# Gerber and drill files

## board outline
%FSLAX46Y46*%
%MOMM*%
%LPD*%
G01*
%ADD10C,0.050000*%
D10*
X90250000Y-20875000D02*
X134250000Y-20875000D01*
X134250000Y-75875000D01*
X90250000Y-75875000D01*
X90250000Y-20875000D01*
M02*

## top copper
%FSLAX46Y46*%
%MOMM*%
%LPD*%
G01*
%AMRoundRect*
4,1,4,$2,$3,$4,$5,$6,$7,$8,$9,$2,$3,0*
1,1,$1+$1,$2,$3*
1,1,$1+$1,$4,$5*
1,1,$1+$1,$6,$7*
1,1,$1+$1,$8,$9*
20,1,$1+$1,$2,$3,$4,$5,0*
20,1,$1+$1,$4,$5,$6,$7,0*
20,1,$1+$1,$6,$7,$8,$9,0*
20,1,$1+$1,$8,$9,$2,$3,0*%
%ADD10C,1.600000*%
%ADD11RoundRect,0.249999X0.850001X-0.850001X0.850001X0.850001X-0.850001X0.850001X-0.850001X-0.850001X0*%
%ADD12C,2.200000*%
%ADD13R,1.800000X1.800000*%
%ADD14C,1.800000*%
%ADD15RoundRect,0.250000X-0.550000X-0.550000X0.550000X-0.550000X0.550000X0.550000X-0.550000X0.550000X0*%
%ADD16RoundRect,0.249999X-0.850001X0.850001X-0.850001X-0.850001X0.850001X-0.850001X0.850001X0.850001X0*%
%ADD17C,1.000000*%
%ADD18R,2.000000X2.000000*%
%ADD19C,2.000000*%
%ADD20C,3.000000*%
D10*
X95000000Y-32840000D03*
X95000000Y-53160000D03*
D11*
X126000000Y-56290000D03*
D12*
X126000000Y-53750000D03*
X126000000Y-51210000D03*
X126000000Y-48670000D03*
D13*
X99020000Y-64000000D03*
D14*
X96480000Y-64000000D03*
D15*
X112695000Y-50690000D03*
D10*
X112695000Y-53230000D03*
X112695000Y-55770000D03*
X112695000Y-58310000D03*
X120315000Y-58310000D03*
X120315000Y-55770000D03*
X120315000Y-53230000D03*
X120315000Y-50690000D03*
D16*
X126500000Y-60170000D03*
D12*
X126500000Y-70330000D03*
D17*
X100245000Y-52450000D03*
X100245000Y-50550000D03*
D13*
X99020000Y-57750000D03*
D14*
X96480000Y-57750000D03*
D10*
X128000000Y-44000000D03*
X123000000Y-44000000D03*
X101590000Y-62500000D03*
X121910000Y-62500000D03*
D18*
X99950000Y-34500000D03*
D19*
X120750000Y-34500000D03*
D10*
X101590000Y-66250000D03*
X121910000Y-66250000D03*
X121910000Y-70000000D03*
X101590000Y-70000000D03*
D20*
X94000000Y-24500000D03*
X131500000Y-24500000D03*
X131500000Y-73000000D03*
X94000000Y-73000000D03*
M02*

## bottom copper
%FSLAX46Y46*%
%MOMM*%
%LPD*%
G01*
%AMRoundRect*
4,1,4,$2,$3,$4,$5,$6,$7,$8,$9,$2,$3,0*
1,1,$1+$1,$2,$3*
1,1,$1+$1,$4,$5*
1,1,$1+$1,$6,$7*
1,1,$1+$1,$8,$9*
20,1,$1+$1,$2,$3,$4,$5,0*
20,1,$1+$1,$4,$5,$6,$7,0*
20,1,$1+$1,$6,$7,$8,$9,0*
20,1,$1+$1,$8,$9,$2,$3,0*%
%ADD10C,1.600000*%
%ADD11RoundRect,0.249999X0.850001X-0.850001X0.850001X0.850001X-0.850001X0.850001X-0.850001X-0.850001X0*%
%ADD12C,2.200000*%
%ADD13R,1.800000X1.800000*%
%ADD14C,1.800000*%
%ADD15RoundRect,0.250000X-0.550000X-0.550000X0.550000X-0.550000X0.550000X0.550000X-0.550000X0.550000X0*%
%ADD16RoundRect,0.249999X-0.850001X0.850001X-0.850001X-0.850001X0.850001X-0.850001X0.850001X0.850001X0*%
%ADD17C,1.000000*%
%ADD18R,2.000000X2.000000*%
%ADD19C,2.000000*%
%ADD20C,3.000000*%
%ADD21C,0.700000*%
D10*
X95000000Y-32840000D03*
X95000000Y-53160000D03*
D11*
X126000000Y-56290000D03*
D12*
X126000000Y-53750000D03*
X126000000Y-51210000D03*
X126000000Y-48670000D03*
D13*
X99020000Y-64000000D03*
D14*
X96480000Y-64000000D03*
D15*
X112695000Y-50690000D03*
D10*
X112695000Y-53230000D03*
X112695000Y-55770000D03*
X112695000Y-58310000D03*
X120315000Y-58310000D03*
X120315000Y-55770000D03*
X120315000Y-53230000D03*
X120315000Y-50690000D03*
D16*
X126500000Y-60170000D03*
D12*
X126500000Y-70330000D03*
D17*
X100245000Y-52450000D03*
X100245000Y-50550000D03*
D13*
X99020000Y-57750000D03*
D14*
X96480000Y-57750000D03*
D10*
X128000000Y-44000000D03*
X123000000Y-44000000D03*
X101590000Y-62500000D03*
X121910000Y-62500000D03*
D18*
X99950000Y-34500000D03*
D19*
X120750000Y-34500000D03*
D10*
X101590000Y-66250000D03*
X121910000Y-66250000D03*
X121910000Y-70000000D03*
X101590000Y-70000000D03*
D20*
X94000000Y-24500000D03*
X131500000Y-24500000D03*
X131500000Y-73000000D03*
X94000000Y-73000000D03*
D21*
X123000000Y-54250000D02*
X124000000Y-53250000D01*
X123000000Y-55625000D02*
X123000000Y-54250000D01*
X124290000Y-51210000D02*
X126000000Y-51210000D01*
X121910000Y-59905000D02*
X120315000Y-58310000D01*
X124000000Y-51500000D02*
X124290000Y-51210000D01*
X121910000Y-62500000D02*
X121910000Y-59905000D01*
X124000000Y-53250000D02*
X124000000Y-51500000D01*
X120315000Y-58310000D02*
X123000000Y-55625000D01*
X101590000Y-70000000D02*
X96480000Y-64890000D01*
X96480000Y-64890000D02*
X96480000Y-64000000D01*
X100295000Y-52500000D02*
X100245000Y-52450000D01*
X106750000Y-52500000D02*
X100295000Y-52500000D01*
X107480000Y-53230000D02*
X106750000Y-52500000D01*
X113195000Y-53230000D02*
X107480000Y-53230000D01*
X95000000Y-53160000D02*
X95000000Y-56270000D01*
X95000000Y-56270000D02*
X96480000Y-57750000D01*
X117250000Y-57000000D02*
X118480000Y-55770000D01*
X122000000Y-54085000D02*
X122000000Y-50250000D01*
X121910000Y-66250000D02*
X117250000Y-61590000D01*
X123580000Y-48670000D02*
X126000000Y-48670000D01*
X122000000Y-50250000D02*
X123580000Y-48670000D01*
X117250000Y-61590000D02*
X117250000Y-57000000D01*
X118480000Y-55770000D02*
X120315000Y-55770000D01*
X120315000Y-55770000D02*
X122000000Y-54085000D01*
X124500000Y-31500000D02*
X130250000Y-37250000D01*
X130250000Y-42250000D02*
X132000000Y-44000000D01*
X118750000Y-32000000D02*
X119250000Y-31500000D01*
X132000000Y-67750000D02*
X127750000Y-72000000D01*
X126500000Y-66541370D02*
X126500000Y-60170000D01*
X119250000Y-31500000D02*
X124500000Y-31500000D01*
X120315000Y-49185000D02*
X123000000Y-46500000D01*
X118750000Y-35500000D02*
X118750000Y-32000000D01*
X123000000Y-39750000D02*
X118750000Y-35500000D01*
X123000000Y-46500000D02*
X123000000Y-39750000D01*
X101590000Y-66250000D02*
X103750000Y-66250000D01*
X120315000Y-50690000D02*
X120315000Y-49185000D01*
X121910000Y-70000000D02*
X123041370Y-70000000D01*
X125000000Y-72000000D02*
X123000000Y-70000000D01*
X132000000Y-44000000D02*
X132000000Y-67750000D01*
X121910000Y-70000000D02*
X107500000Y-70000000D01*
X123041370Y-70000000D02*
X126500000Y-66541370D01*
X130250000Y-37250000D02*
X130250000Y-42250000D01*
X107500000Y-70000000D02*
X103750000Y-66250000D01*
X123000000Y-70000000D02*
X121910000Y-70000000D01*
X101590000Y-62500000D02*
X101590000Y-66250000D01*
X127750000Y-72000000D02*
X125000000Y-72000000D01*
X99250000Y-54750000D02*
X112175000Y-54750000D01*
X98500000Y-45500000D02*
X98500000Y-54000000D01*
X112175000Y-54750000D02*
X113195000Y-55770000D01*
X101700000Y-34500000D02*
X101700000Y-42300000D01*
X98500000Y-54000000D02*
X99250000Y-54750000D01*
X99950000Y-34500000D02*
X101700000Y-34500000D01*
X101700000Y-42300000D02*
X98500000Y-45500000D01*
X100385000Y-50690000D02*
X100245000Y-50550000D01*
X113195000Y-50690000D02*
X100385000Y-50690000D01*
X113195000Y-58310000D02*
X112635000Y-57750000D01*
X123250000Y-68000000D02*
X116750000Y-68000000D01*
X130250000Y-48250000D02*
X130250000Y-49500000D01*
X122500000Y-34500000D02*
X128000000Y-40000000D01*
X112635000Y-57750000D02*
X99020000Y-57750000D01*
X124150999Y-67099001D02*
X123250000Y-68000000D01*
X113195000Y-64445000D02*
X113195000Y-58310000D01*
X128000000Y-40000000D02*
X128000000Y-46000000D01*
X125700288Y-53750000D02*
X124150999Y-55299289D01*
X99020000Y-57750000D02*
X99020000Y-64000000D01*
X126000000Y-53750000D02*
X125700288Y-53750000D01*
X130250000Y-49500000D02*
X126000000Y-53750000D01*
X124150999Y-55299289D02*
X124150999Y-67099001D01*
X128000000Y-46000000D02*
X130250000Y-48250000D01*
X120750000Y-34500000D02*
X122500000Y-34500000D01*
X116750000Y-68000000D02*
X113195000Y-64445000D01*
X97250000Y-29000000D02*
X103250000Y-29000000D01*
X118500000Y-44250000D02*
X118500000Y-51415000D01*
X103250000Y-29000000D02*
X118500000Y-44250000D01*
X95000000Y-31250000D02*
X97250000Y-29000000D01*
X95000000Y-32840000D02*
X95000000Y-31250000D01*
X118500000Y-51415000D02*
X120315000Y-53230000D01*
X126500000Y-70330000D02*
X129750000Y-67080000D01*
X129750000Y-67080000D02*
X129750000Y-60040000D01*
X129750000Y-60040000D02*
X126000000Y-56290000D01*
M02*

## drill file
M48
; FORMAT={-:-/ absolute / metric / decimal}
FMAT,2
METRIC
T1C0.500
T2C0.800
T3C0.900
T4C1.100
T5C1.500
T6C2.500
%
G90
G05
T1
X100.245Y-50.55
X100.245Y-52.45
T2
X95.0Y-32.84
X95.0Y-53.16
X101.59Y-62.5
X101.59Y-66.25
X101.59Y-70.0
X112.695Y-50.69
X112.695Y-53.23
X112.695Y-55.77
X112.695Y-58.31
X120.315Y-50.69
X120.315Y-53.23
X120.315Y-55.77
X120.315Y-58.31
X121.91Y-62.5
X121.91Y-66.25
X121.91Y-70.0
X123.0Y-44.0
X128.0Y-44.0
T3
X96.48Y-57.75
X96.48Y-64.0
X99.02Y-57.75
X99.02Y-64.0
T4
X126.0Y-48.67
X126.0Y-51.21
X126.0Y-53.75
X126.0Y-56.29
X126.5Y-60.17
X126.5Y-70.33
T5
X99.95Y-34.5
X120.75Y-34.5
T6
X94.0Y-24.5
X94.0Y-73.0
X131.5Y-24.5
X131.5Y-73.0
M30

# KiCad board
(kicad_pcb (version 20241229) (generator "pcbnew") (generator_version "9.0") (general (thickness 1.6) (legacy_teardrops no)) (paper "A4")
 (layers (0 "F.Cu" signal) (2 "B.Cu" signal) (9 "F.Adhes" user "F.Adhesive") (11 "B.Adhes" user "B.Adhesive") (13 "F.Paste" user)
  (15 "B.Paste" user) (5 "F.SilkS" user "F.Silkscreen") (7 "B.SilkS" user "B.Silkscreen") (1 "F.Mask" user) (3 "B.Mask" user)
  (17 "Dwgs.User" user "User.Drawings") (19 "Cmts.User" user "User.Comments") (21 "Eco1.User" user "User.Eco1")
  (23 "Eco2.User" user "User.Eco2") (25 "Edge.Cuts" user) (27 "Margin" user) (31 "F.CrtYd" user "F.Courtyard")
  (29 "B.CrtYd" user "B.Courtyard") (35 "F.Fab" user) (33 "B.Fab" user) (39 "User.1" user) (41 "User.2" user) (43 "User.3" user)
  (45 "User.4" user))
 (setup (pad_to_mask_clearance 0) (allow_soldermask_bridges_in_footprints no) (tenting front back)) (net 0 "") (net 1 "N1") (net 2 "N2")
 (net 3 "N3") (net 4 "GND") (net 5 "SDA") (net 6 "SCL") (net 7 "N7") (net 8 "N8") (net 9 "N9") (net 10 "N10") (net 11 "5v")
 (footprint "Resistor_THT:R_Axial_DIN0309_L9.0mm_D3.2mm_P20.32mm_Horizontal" (layer "F.Cu") (at 95 32.84 -90)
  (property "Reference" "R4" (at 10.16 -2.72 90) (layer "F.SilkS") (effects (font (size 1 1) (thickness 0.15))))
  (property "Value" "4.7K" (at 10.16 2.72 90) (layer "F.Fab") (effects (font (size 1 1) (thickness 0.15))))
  (pad "1" thru_hole circle (at 0 0 270) (size 1.6 1.6) (drill 0.8) (layers "*.Cu" "*.Mask") (remove_unused_layers no) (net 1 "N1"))
  (pad "2" thru_hole circle (at 20.32 0 270) (size 1.6 1.6) (drill 0.8) (layers "*.Cu" "*.Mask") (remove_unused_layers no) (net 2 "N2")))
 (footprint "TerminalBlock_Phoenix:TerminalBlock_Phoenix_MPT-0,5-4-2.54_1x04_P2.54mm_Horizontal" (layer "F.Cu") (at 126 56.29 90)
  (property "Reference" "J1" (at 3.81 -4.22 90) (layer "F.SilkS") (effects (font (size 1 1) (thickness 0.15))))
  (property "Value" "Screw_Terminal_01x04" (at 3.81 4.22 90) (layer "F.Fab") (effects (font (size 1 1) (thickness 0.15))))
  (pad "1" thru_hole roundrect (at 0 0 90) (size 2.2 2.2) (drill 1.1) (layers "*.Cu" "*.Mask") (remove_unused_layers no)
   (roundrect_rratio 0.113636) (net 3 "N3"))
  (pad "2" thru_hole circle (at 2.54 0 90) (size 2.2 2.2) (drill 1.1) (layers "*.Cu" "*.Mask") (remove_unused_layers no) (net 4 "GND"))
  (pad "3" thru_hole circle (at 5.08 0 90) (size 2.2 2.2) (drill 1.1) (layers "*.Cu" "*.Mask") (remove_unused_layers no) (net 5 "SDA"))
  (pad "4" thru_hole circle (at 7.62 0 90) (size 2.2 2.2) (drill 1.1) (layers "*.Cu" "*.Mask") (remove_unused_layers no) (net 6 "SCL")))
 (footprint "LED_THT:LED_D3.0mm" (layer "F.Cu") (at 99.02 64 180)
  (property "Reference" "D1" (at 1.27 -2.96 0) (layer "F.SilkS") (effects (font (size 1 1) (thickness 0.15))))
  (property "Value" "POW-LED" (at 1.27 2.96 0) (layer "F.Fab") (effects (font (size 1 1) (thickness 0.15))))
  (pad "1" thru_hole rect (at 0 0 180) (size 1.8 1.8) (drill 0.9) (layers "*.Cu" "*.Mask") (remove_unused_layers no) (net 4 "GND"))
  (pad "2" thru_hole circle (at 2.54 0 180) (size 1.8 1.8) (drill 0.9) (layers "*.Cu" "*.Mask") (remove_unused_layers no) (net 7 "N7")))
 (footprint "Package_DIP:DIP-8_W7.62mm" (layer "F.Cu") (at 112.695 50.69)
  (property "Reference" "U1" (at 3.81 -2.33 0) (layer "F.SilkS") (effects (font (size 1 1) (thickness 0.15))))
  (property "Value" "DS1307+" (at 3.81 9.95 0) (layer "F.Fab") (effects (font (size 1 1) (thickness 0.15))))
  (pad "1" thru_hole roundrect (at 0 0) (size 1.6 1.6) (drill 0.8) (layers "*.Cu" "*.Mask") (remove_unused_layers no)
   (roundrect_rratio 0.15625) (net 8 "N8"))
  (pad "2" thru_hole circle (at 0 2.54) (size 1.6 1.6) (drill 0.8) (layers "*.Cu" "*.Mask") (remove_unused_layers no) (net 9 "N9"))
  (pad "3" thru_hole circle (at 0 5.08) (size 1.6 1.6) (drill 0.8) (layers "*.Cu" "*.Mask") (remove_unused_layers no) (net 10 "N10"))
  (pad "4" thru_hole circle (at 0 7.62) (size 1.6 1.6) (drill 0.8) (layers "*.Cu" "*.Mask") (remove_unused_layers no) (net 4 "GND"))
  (pad "5" thru_hole circle (at 7.62 7.62) (size 1.6 1.6) (drill 0.8) (layers "*.Cu" "*.Mask") (remove_unused_layers no) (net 5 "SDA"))
  (pad "6" thru_hole circle (at 7.62 5.08) (size 1.6 1.6) (drill 0.8) (layers "*.Cu" "*.Mask") (remove_unused_layers no) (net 6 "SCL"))
  (pad "7" thru_hole circle (at 7.62 2.54) (size 1.6 1.6) (drill 0.8) (layers "*.Cu" "*.Mask") (remove_unused_layers no) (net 1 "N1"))
  (pad "8" thru_hole circle (at 7.62 0) (size 1.6 1.6) (drill 0.8) (layers "*.Cu" "*.Mask") (remove_unused_layers no) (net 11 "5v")))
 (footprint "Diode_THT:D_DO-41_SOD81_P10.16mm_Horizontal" (layer "F.Cu") (at 126.5 60.17 -90)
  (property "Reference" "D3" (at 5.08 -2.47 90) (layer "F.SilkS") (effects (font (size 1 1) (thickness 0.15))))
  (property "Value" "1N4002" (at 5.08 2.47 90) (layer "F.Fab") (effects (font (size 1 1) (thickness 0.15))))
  (pad "1" thru_hole roundrect (at 0 0 270) (size 2.2 2.2) (drill 1.1) (layers "*.Cu" "*.Mask") (remove_unused_layers no)
   (roundrect_rratio 0.113636) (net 11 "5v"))
  (pad "2" thru_hole circle (at 10.16 0 270) (size 2.2 2.2) (drill 1.1) (layers "*.Cu" "*.Mask") (remove_unused_layers no) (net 3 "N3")))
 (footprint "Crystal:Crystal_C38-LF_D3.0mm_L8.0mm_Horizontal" (layer "F.Cu") (at 100.245 52.45 90)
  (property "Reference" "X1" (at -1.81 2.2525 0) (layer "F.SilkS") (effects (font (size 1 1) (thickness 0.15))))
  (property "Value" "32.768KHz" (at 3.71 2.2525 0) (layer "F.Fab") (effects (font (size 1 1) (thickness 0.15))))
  (pad "1" thru_hole circle (at 0 0 90) (size 1 1) (drill 0.5) (layers "*.Cu" "*.Mask") (remove_unused_layers no) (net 9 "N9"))
  (pad "2" thru_hole circle (at 1.9 0 90) (size 1 1) (drill 0.5) (layers "*.Cu" "*.Mask") (remove_unused_layers no) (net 8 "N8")))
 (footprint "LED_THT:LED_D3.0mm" (layer "F.Cu") (at 99.02 57.75 180)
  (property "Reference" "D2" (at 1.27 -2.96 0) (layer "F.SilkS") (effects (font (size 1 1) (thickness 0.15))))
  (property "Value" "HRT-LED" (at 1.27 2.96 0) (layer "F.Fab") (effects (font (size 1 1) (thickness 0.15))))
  (pad "1" thru_hole rect (at 0 0 180) (size 1.8 1.8) (drill 0.9) (layers "*.Cu" "*.Mask") (remove_unused_layers no) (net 4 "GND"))
  (pad "2" thru_hole circle (at 2.54 0 180) (size 1.8 1.8) (drill 0.9) (layers "*.Cu" "*.Mask") (remove_unused_layers no) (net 2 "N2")))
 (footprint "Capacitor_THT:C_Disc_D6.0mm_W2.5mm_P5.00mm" (layer "F.Cu") (at 128 44 180)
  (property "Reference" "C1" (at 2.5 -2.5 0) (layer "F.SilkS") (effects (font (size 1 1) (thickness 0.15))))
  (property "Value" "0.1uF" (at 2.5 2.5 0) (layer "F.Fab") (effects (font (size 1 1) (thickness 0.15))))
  (pad "1" thru_hole circle (at 0 0 180) (size 1.6 1.6) (drill 0.8) (layers "*.Cu" "*.Mask") (remove_unused_layers no) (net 4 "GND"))
  (pad "2" thru_hole circle (at 5 0 180) (size 1.6 1.6) (drill 0.8) (layers "*.Cu" "*.Mask") (remove_unused_layers no) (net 11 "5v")))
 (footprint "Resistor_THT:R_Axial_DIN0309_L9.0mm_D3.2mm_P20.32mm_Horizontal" (layer "F.Cu") (at 101.59 62.5)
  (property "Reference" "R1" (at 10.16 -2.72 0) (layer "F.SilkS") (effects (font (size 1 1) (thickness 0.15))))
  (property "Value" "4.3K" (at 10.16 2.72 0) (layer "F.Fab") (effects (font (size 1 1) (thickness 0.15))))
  (pad "1" thru_hole circle (at 0 0) (size 1.6 1.6) (drill 0.8) (layers "*.Cu" "*.Mask") (remove_unused_layers no) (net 11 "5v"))
  (pad "2" thru_hole circle (at 20.32 0) (size 1.6 1.6) (drill 0.8) (layers "*.Cu" "*.Mask") (remove_unused_layers no) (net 5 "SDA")))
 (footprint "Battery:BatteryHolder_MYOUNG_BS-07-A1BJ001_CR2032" (layer "F.Cu") (at 99.95 34.5)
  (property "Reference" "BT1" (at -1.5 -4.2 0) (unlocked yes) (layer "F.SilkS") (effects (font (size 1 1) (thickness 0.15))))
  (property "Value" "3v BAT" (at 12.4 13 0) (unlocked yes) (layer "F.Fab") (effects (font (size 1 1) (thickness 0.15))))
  (pad "1" thru_hole rect (at 0 0 180) (size 2 2) (drill 1.5) (layers "*.Cu" "*.Mask") (remove_unused_layers no) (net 10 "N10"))
  (pad "2" thru_hole circle (at 20.8 0 180) (size 2 2) (drill 1.5) (layers "*.Cu" "*.Mask") (remove_unused_layers no) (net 4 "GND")))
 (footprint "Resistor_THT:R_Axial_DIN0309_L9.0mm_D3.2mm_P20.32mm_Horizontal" (layer "F.Cu") (at 101.59 66.25)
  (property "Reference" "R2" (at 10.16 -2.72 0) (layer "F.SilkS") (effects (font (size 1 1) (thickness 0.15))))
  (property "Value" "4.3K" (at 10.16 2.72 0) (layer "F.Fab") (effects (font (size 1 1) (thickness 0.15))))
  (pad "1" thru_hole circle (at 0 0) (size 1.6 1.6) (drill 0.8) (layers "*.Cu" "*.Mask") (remove_unused_layers no) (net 11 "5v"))
  (pad "2" thru_hole circle (at 20.32 0) (size 1.6 1.6) (drill 0.8) (layers "*.Cu" "*.Mask") (remove_unused_layers no) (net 6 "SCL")))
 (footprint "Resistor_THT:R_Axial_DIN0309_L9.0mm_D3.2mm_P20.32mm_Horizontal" (layer "F.Cu") (at 121.91 70 180)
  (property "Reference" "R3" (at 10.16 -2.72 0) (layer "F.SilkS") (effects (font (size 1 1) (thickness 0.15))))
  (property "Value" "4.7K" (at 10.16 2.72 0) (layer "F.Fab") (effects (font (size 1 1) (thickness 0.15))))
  (pad "1" thru_hole circle (at 0 0 180) (size 1.6 1.6) (drill 0.8) (layers "*.Cu" "*.Mask") (remove_unused_layers no) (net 11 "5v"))
  (pad "2" thru_hole circle (at 20.32 0 180) (size 1.6 1.6) (drill 0.8) (layers "*.Cu" "*.Mask") (remove_unused_layers no) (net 7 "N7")))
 (gr_rect (start 90.25 20.875) (end 134.25 75.875) (stroke (width 0.05) (type default)) (fill no) (layer "Edge.Cuts"))
 (via (at 94 24.5) (size 3) (drill 2.5) (layers "F.Cu" "B.Cu") (tenting front back) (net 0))
 (via (at 131.5 24.5) (size 3) (drill 2.5) (layers "F.Cu" "B.Cu") (tenting front back) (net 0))
 (via (at 131.5 73) (size 3) (drill 2.5) (layers "F.Cu" "B.Cu") (tenting front back) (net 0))
 (via (at 94 73) (size 3) (drill 2.5) (layers "F.Cu" "B.Cu") (tenting front back) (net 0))
 (segment (start 123 54.25) (end 124 53.25) (width 0.7) (layer "B.Cu") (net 5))
 (segment (start 123 55.625) (end 123 54.25) (width 0.7) (layer "B.Cu") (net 5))
 (segment (start 124.29 51.21) (end 126 51.21) (width 0.7) (layer "B.Cu") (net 5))
 (segment (start 121.91 59.905) (end 120.315 58.31) (width 0.7) (layer "B.Cu") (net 5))
 (segment (start 124 51.5) (end 124.29 51.21) (width 0.7) (layer "B.Cu") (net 5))
 (segment (start 121.91 62.5) (end 121.91 59.905) (width 0.7) (layer "B.Cu") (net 5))
 (segment (start 124 53.25) (end 124 51.5) (width 0.7) (layer "B.Cu") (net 5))
 (segment (start 120.315 58.31) (end 123 55.625) (width 0.7) (layer "B.Cu") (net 5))
 (segment (start 101.59 70) (end 96.48 64.89) (width 0.7) (layer "B.Cu") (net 7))
 (segment (start 96.48 64.89) (end 96.48 64) (width 0.7) (layer "B.Cu") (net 7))
 (segment (start 100.295 52.5) (end 100.245 52.45) (width 0.7) (layer "B.Cu") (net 9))
 (segment (start 106.75 52.5) (end 100.295 52.5) (width 0.7) (layer "B.Cu") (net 9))
 (segment (start 107.48 53.23) (end 106.75 52.5) (width 0.7) (layer "B.Cu") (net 9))
 (segment (start 113.195 53.23) (end 107.48 53.23) (width 0.7) (layer "B.Cu") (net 9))
 (segment (start 95 53.16) (end 95 56.27) (width 0.7) (layer "B.Cu") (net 2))
 (segment (start 95 56.27) (end 96.48 57.75) (width 0.7) (layer "B.Cu") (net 2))
 (segment (start 117.25 57) (end 118.48 55.77) (width 0.7) (layer "B.Cu") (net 6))
 (segment (start 122 54.085) (end 122 50.25) (width 0.7) (layer "B.Cu") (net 6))
 (segment (start 121.91 66.25) (end 117.25 61.59) (width 0.7) (layer "B.Cu") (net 6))
 (segment (start 123.58 48.67) (end 126 48.67) (width 0.7) (layer "B.Cu") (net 6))
 (segment (start 122 50.25) (end 123.58 48.67) (width 0.7) (layer "B.Cu") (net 6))
 (segment (start 117.25 61.59) (end 117.25 57) (width 0.7) (layer "B.Cu") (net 6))
 (segment (start 118.48 55.77) (end 120.315 55.77) (width 0.7) (layer "B.Cu") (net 6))
 (segment (start 120.315 55.77) (end 122 54.085) (width 0.7) (layer "B.Cu") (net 6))
 (segment (start 124.5 31.5) (end 130.25 37.25) (width 0.7) (layer "B.Cu") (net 11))
 (segment (start 130.25 42.25) (end 132 44) (width 0.7) (layer "B.Cu") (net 11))
 (segment (start 118.75 32) (end 119.25 31.5) (width 0.7) (layer "B.Cu") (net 11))
 (segment (start 132 67.75) (end 127.75 72) (width 0.7) (layer "B.Cu") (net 11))
 (segment (start 126.5 66.54137) (end 126.5 60.17) (width 0.7) (layer "B.Cu") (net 11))
 (segment (start 119.25 31.5) (end 124.5 31.5) (width 0.7) (layer "B.Cu") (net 11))
 (segment (start 120.315 49.185) (end 123 46.5) (width 0.7) (layer "B.Cu") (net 11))
 (segment (start 118.75 35.5) (end 118.75 32) (width 0.7) (layer "B.Cu") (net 11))
 (segment (start 123 39.75) (end 118.75 35.5) (width 0.7) (layer "B.Cu") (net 11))
 (segment (start 123 46.5) (end 123 39.75) (width 0.7) (layer "B.Cu") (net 11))
 (segment (start 101.59 66.25) (end 103.75 66.25) (width 0.7) (layer "B.Cu") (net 11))
 (segment (start 120.315 50.69) (end 120.315 49.185) (width 0.7) (layer "B.Cu") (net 11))
 (segment (start 121.91 70) (end 123.04137 70) (width 0.7) (layer "B.Cu") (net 11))
 (segment (start 125 72) (end 123 70) (width 0.7) (layer "B.Cu") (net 11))
 (segment (start 132 44) (end 132 67.75) (width 0.7) (layer "B.Cu") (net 11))
 (segment (start 121.91 70) (end 107.5 70) (width 0.7) (layer "B.Cu") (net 11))
 (segment (start 123.04137 70) (end 126.5 66.54137) (width 0.7) (layer "B.Cu") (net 11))
 (segment (start 130.25 37.25) (end 130.25 42.25) (width 0.7) (layer "B.Cu") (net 11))
 (segment (start 107.5 70) (end 103.75 66.25) (width 0.7) (layer "B.Cu") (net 11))
 (segment (start 123 70) (end 121.91 70) (width 0.7) (layer "B.Cu") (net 11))
 (segment (start 101.59 62.5) (end 101.59 66.25) (width 0.7) (layer "B.Cu") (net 11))
 (segment (start 127.75 72) (end 125 72) (width 0.7) (layer "B.Cu") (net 11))
 (segment (start 99.25 54.75) (end 112.175 54.75) (width 0.7) (layer "B.Cu") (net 10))
 (segment (start 98.5 45.5) (end 98.5 54) (width 0.7) (layer "B.Cu") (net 10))
 (segment (start 112.175 54.75) (end 113.195 55.77) (width 0.7) (layer "B.Cu") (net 10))
 (segment (start 101.7 34.5) (end 101.7 42.3) (width 0.7) (layer "B.Cu") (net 10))
 (segment (start 98.5 54) (end 99.25 54.75) (width 0.7) (layer "B.Cu") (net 10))
 (segment (start 99.95 34.5) (end 101.7 34.5) (width 0.7) (layer "B.Cu") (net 10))
 (segment (start 101.7 42.3) (end 98.5 45.5) (width 0.7) (layer "B.Cu") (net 10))
 (segment (start 100.385 50.69) (end 100.245 50.55) (width 0.7) (layer "B.Cu") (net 8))
 (segment (start 113.195 50.69) (end 100.385 50.69) (width 0.7) (layer "B.Cu") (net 8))
 (segment (start 113.195 58.31) (end 112.635 57.75) (width 0.7) (layer "B.Cu") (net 4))
 (segment (start 123.25 68) (end 116.75 68) (width 0.7) (layer "B.Cu") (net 4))
 (segment (start 130.25 48.25) (end 130.25 49.5) (width 0.7) (layer "B.Cu") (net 4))
 (segment (start 122.5 34.5) (end 128 40) (width 0.7) (layer "B.Cu") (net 4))
 (segment (start 112.635 57.75) (end 99.02 57.75) (width 0.7) (layer "B.Cu") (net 4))
 (segment (start 124.150999 67.099001) (end 123.25 68) (width 0.7) (layer "B.Cu") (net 4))
 (segment (start 113.195 64.445) (end 113.195 58.31) (width 0.7) (layer "B.Cu") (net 4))
 (segment (start 128 40) (end 128 46) (width 0.7) (layer "B.Cu") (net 4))
 (segment (start 125.700288 53.75) (end 124.150999 55.299289) (width 0.7) (layer "B.Cu") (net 4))
 (segment (start 99.02 57.75) (end 99.02 64) (width 0.7) (layer "B.Cu") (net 4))
 (segment (start 126 53.75) (end 125.700288 53.75) (width 0.7) (layer "B.Cu") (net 4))
 (segment (start 130.25 49.5) (end 126 53.75) (width 0.7) (layer "B.Cu") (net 4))
 (segment (start 124.150999 55.299289) (end 124.150999 67.099001) (width 0.7) (layer "B.Cu") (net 4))
 (segment (start 128 46) (end 130.25 48.25) (width 0.7) (layer "B.Cu") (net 4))
 (segment (start 120.75 34.5) (end 122.5 34.5) (width 0.7) (layer "B.Cu") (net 4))
 (segment (start 116.75 68) (end 113.195 64.445) (width 0.7) (layer "B.Cu") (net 4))
 (segment (start 97.25 29) (end 103.25 29) (width 0.7) (layer "B.Cu") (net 1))
 (segment (start 118.5 44.25) (end 118.5 51.415) (width 0.7) (layer "B.Cu") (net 1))
 (segment (start 103.25 29) (end 118.5 44.25) (width 0.7) (layer "B.Cu") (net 1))
 (segment (start 95 31.25) (end 97.25 29) (width 0.7) (layer "B.Cu") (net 1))
 (segment (start 95 32.84) (end 95 31.25) (width 0.7) (layer "B.Cu") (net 1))
 (segment (start 118.5 51.415) (end 120.315 53.23) (width 0.7) (layer "B.Cu") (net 1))
 (segment (start 126.5 70.33) (end 129.75 67.08) (width 0.7) (layer "B.Cu") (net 3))
 (segment (start 129.75 67.08) (end 129.75 60.04) (width 0.7) (layer "B.Cu") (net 3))
 (segment (start 129.75 60.04) (end 126 56.29) (width 0.7) (layer "B.Cu") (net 3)))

